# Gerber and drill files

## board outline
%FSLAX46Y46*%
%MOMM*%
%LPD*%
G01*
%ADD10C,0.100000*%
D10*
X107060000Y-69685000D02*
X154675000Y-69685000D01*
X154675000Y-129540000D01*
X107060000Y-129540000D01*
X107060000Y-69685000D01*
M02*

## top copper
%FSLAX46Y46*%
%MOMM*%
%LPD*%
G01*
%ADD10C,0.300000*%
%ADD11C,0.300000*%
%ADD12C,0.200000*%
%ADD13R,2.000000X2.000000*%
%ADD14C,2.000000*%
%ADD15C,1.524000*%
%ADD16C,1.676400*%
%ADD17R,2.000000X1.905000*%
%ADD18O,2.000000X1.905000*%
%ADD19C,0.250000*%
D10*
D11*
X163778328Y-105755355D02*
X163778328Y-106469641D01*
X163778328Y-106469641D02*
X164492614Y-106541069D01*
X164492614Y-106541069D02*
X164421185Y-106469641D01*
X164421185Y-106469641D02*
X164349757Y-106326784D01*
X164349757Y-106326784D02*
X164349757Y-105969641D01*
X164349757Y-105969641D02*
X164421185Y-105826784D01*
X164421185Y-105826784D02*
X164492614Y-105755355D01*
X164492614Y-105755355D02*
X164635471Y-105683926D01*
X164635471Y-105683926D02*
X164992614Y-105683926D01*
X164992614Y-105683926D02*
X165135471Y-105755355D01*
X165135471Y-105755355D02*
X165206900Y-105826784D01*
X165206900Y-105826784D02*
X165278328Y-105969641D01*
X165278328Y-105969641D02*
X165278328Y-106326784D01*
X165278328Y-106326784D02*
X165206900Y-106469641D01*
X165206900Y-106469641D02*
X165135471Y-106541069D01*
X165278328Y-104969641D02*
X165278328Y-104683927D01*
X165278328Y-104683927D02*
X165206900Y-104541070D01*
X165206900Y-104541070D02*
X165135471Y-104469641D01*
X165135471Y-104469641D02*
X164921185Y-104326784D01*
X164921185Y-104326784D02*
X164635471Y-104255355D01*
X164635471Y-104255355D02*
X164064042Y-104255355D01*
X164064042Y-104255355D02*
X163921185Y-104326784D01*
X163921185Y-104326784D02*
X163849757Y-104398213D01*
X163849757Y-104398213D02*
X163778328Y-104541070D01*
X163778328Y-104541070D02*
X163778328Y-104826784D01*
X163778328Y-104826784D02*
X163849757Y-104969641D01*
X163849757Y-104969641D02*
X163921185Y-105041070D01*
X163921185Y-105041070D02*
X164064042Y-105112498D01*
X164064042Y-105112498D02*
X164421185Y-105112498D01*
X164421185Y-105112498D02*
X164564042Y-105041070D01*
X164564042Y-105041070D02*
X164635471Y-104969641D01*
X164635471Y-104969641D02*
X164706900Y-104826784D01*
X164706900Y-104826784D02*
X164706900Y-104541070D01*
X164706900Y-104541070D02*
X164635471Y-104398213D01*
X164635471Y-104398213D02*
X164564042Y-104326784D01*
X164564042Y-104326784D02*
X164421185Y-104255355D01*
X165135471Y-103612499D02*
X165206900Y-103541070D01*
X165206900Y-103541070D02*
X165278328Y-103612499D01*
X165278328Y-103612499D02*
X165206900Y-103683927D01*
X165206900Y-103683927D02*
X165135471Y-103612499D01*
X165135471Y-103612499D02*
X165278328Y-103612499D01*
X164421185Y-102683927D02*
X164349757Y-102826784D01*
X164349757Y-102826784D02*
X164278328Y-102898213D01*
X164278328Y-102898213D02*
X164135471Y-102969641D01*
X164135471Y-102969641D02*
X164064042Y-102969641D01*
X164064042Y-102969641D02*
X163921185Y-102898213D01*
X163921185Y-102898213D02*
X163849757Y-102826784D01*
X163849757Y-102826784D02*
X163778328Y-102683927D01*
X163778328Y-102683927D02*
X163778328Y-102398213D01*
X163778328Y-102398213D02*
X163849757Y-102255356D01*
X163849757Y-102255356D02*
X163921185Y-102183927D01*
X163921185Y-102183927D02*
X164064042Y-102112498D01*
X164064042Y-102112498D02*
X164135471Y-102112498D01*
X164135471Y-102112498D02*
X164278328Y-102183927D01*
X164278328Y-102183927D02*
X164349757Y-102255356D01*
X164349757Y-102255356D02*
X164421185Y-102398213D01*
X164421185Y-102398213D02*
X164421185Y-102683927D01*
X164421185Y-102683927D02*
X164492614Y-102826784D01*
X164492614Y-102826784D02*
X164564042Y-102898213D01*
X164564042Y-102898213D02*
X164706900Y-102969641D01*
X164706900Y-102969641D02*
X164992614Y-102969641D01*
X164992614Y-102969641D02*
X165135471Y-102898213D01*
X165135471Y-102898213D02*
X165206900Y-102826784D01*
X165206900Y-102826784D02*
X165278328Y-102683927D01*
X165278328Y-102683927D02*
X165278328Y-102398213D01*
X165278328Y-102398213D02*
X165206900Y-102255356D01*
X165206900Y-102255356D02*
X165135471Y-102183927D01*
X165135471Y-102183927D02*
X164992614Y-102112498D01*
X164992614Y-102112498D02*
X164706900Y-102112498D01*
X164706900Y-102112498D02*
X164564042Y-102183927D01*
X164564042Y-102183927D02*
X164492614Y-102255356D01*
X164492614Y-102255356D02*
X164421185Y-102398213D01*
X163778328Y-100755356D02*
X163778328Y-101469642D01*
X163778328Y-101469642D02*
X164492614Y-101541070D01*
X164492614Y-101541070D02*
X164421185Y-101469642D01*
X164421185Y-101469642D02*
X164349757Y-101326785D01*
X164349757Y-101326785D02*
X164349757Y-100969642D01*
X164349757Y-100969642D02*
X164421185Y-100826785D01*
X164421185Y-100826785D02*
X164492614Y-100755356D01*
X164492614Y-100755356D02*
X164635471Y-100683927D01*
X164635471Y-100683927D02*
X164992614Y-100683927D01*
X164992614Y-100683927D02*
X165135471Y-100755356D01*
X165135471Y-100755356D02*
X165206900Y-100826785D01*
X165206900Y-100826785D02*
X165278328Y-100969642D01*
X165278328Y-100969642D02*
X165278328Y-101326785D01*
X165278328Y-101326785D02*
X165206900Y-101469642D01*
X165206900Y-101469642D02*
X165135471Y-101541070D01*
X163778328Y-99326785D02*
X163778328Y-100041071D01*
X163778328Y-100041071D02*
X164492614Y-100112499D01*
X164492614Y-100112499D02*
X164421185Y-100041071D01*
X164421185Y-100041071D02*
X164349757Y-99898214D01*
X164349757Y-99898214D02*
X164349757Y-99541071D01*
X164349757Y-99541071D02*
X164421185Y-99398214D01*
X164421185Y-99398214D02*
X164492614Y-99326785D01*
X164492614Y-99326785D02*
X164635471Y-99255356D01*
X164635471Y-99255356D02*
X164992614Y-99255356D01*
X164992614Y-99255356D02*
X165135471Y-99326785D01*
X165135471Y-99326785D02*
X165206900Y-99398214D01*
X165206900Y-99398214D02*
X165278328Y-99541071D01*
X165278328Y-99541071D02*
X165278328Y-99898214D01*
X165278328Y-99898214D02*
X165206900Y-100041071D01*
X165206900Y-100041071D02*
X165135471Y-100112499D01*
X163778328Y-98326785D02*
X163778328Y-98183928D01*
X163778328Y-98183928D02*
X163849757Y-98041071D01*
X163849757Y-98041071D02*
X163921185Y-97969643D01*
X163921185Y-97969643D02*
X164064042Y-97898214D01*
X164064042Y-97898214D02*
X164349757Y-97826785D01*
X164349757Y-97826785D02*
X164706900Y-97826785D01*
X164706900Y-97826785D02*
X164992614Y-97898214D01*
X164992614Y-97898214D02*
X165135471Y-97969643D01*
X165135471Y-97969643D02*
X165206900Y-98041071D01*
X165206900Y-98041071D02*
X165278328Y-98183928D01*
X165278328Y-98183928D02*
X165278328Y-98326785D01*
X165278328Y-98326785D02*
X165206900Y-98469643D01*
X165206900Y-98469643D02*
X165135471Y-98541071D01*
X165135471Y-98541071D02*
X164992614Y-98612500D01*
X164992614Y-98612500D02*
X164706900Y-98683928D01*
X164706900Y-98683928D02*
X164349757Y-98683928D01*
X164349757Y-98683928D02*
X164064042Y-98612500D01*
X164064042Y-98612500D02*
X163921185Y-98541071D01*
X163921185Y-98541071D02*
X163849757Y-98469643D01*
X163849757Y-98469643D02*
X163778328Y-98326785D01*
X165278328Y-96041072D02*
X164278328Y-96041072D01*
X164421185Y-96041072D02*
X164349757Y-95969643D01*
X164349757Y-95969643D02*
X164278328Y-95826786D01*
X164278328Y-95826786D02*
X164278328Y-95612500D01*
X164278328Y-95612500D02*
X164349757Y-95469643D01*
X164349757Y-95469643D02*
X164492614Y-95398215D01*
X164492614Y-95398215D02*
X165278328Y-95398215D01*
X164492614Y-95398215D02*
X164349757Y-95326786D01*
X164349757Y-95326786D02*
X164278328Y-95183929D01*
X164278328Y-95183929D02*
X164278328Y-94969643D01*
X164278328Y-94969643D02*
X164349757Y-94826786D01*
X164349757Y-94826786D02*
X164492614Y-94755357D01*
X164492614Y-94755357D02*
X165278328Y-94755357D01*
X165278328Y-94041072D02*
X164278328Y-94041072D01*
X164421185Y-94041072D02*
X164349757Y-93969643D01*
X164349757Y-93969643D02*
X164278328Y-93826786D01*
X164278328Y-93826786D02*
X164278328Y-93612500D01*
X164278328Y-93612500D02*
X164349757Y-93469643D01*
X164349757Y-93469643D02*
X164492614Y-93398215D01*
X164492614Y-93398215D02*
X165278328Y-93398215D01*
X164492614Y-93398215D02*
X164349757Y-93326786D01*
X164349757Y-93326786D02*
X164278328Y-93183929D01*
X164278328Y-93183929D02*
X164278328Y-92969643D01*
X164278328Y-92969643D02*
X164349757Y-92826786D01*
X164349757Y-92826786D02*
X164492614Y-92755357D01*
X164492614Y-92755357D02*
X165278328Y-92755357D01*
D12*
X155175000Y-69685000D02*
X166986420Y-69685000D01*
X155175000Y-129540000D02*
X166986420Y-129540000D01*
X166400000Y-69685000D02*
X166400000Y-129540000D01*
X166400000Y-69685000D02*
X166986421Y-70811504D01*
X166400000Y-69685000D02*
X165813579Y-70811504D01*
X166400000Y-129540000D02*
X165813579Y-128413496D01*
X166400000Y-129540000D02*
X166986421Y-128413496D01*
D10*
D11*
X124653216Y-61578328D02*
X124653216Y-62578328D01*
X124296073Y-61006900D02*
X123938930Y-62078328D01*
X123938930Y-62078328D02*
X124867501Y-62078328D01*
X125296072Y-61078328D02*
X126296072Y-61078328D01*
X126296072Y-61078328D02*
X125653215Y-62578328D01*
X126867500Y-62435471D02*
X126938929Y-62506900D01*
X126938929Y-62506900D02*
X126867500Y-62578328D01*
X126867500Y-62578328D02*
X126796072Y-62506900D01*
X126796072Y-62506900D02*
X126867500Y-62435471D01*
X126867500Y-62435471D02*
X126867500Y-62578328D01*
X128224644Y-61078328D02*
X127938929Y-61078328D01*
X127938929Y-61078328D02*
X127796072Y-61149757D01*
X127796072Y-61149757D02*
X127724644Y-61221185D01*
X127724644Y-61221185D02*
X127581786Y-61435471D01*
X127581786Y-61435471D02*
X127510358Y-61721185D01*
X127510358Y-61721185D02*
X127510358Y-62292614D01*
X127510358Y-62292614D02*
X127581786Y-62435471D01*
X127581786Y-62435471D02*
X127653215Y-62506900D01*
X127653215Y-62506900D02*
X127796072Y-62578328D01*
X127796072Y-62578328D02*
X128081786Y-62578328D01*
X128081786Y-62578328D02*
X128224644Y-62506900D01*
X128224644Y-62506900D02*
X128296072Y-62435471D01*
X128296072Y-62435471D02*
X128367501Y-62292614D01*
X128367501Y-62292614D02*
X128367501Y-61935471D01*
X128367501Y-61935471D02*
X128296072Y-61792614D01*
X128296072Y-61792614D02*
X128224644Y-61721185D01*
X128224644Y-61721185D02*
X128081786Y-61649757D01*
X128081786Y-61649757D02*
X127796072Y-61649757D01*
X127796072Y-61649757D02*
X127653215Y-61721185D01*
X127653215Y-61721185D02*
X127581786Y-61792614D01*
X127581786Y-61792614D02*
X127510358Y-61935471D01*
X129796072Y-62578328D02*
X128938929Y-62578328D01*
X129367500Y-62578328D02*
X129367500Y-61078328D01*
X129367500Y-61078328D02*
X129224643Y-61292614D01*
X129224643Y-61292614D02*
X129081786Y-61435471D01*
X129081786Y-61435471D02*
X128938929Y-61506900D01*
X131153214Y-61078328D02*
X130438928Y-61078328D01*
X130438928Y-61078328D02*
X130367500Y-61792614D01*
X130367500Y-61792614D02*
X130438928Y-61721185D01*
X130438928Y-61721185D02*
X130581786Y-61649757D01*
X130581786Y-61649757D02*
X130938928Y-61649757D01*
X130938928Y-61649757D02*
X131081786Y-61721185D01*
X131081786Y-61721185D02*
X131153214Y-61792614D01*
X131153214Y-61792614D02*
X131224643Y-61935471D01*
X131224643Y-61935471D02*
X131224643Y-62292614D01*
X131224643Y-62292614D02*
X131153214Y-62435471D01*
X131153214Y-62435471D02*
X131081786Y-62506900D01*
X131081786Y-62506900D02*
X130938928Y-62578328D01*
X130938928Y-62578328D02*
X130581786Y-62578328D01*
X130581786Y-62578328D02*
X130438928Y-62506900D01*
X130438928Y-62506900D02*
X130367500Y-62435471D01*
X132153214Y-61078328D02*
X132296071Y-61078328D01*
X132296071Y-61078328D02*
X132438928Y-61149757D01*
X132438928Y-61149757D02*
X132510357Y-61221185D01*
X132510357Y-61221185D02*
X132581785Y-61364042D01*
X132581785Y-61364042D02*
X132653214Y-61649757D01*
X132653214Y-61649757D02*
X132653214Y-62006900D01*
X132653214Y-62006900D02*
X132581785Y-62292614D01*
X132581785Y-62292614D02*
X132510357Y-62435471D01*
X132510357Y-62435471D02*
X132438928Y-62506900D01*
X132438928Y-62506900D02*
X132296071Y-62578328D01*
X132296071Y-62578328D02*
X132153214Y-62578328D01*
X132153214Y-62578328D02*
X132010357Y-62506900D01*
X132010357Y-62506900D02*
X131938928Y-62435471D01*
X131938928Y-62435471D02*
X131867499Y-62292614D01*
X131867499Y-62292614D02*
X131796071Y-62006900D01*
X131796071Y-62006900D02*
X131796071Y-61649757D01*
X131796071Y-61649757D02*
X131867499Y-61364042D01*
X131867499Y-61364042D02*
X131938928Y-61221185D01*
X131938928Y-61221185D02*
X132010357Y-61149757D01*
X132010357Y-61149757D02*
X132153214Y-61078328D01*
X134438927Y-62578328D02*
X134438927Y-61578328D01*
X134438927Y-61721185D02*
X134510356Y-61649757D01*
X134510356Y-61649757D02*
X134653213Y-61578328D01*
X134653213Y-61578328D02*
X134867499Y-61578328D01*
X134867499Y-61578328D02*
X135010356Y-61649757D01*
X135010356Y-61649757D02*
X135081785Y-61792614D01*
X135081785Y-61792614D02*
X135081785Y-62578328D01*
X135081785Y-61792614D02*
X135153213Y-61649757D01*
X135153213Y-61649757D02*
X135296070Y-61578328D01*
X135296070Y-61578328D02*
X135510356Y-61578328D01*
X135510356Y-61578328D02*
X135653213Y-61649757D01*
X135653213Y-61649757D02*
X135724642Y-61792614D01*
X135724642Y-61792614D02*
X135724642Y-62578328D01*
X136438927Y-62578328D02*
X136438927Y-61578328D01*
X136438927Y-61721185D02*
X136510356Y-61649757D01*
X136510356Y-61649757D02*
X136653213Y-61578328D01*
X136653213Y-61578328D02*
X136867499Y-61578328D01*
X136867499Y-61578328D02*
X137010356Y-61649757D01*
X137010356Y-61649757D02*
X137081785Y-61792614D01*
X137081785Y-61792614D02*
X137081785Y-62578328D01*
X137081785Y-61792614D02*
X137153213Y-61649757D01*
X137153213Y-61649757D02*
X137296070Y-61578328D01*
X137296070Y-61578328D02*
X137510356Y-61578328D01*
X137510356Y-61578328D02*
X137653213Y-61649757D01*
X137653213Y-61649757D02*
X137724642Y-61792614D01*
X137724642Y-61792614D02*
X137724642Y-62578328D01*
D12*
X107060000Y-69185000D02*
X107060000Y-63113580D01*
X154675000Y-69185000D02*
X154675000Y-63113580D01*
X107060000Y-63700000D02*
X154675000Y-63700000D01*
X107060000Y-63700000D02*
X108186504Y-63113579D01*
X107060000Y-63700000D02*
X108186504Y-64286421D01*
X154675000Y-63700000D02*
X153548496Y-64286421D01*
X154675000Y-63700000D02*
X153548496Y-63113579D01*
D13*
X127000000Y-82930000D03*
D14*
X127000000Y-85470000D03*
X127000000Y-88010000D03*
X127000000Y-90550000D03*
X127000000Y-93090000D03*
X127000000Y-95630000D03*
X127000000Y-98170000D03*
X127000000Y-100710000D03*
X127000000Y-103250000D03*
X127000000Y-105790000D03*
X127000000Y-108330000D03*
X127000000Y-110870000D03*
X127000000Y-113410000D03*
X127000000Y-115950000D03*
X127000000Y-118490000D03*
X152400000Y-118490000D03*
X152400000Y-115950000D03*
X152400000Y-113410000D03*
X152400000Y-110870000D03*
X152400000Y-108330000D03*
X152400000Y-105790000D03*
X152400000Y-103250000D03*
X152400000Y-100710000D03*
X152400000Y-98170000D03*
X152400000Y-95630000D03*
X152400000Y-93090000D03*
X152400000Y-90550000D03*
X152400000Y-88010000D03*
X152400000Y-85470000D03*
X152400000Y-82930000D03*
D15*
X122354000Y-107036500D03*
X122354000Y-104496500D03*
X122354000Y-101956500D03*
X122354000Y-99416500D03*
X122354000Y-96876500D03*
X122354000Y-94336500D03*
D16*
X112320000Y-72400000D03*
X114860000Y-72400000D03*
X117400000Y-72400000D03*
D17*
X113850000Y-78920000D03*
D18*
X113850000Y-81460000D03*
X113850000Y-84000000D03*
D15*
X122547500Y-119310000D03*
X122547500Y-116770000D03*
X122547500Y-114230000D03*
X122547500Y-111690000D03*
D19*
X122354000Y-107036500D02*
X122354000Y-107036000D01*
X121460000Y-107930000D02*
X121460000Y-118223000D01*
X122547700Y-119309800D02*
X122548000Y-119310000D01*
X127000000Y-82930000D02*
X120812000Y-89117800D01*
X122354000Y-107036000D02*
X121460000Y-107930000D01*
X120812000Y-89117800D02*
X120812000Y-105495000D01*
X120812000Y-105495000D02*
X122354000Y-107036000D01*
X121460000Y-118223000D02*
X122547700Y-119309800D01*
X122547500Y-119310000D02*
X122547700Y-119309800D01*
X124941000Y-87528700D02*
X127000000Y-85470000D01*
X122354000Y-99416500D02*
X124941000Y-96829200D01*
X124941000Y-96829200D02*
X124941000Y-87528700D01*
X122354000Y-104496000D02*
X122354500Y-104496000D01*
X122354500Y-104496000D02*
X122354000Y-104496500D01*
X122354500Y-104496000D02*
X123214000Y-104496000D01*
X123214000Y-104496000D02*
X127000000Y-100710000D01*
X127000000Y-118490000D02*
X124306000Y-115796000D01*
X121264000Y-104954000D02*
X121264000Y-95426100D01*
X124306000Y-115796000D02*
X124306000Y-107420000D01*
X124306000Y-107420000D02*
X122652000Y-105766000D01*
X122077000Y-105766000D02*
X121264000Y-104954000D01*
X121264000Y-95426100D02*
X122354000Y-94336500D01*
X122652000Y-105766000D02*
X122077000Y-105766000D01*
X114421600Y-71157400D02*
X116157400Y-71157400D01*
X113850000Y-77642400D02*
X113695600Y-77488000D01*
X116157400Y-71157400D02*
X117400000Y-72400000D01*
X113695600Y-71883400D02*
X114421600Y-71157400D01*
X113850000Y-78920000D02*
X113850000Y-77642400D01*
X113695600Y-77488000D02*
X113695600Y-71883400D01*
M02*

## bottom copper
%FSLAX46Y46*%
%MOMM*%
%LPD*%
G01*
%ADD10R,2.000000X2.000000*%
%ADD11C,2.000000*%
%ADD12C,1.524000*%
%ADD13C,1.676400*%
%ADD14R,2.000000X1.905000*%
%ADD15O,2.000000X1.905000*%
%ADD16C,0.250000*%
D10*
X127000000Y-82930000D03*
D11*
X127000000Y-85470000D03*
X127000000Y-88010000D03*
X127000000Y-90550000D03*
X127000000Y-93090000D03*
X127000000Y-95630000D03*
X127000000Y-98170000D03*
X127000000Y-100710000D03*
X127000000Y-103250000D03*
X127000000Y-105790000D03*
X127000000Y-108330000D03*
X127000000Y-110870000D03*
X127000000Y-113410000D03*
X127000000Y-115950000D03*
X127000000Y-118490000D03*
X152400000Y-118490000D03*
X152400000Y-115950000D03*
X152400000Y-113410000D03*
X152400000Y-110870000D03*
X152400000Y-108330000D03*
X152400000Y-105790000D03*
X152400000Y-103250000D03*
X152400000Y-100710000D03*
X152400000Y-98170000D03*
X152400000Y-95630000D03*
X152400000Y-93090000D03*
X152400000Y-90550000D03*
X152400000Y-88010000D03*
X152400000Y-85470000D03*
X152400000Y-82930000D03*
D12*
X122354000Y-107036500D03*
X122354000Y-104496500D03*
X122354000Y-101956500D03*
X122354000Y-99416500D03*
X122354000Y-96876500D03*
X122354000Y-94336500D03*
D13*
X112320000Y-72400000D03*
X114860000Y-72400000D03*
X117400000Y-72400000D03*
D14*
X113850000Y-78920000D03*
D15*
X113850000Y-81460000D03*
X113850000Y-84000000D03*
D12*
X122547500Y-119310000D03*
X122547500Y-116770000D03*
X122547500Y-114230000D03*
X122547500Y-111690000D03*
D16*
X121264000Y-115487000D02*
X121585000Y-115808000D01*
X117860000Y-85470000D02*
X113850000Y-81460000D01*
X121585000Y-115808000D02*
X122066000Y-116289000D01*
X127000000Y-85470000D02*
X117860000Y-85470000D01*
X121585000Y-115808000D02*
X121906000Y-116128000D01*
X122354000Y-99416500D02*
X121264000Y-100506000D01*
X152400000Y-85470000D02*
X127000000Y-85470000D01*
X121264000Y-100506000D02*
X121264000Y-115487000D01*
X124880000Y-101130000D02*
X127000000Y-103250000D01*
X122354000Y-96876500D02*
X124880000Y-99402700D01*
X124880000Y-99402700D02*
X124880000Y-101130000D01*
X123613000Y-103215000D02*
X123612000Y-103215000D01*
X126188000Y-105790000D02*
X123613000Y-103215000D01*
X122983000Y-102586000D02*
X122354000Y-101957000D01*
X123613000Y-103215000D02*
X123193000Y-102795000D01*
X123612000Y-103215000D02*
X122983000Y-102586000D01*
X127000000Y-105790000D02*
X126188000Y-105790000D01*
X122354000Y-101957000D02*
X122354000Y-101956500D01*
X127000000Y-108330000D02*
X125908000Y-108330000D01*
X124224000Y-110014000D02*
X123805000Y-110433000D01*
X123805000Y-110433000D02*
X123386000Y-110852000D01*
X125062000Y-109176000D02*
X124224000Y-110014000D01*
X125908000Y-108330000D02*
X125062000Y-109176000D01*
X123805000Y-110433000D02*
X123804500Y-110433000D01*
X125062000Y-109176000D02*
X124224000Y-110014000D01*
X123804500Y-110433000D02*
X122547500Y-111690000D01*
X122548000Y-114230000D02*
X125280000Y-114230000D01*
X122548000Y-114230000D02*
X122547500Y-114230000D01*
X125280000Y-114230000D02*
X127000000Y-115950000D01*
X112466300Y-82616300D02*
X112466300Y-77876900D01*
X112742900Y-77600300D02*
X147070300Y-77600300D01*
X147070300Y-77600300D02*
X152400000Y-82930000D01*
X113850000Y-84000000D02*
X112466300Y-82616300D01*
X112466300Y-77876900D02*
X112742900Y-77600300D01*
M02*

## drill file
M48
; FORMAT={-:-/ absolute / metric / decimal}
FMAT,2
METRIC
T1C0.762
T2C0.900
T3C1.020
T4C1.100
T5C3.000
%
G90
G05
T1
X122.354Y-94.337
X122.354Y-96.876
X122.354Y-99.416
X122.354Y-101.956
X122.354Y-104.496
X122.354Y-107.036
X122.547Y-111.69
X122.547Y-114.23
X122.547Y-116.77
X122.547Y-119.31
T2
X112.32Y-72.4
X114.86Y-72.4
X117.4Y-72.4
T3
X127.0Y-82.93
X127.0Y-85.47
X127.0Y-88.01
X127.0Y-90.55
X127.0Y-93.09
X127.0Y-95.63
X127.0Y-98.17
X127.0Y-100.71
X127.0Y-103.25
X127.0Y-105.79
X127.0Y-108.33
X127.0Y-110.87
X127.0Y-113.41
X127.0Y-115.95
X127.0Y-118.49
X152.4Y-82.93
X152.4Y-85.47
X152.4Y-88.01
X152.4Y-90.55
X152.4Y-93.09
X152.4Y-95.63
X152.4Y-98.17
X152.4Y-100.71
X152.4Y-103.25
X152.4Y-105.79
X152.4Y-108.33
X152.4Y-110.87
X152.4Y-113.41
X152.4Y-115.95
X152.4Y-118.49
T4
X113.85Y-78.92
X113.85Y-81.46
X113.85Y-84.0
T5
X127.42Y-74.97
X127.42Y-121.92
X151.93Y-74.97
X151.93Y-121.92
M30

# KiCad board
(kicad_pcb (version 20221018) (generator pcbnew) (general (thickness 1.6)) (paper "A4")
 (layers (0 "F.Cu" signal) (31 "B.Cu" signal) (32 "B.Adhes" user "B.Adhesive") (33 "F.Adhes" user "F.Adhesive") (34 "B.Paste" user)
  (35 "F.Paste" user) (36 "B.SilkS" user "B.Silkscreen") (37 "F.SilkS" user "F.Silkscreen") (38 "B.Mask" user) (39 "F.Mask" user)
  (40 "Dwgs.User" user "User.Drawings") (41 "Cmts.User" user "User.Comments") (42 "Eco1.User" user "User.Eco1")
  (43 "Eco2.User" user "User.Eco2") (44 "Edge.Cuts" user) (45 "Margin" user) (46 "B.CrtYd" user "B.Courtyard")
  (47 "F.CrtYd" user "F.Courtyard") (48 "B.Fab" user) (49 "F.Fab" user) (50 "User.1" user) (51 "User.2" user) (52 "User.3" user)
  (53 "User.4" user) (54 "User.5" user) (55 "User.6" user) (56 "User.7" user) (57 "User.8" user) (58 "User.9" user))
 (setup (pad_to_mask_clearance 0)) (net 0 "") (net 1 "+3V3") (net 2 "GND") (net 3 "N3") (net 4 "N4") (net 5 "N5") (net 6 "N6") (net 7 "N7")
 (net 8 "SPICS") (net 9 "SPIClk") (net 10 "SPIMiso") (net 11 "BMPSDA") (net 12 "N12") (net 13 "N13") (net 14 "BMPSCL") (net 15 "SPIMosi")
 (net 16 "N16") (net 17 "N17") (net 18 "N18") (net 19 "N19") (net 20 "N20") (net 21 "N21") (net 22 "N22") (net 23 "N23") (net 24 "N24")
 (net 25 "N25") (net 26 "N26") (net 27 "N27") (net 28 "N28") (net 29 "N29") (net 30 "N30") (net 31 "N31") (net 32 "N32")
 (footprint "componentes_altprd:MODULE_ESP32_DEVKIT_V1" (layer "F.Cu") (at 139.7 98.445)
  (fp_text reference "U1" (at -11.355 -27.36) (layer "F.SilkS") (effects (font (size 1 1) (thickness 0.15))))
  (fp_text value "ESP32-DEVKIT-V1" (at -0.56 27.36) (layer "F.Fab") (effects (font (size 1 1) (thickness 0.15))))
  (pad "" np_thru_hole circle (at -12.28 -23.475) (size 3 3) (drill 3) (layers "*.Cu" "*.Mask"))
  (pad "" np_thru_hole circle (at -12.28 23.475) (size 3 3) (drill 3) (layers "*.Cu" "*.Mask"))
  (pad "" np_thru_hole circle (at 12.23 -23.475) (size 3 3) (drill 3) (layers "*.Cu" "*.Mask"))
  (pad "" np_thru_hole circle (at 12.23 23.475) (size 3 3) (drill 3) (layers "*.Cu" "*.Mask"))
  (pad "1" thru_hole rect (at -12.7 -15.515) (size 2 2) (drill 1.02) (layers "*.Cu" "*.Mask") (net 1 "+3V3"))
  (pad "2" thru_hole circle (at -12.7 -12.975) (size 2 2) (drill 1.02) (layers "*.Cu" "*.Mask") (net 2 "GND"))
  (pad "3" thru_hole circle (at -12.7 -10.435) (size 2 2) (drill 1.02) (layers "*.Cu" "*.Mask") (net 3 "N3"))
  (pad "4" thru_hole circle (at -12.7 -7.895) (size 2 2) (drill 1.02) (layers "*.Cu" "*.Mask") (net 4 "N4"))
  (pad "5" thru_hole circle (at -12.7 -5.355) (size 2 2) (drill 1.02) (layers "*.Cu" "*.Mask") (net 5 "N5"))
  (pad "6" thru_hole circle (at -12.7 -2.815) (size 2 2) (drill 1.02) (layers "*.Cu" "*.Mask") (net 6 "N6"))
  (pad "7" thru_hole circle (at -12.7 -0.275) (size 2 2) (drill 1.02) (layers "*.Cu" "*.Mask") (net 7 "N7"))
  (pad "8" thru_hole circle (at -12.7 2.265) (size 2 2) (drill 1.02) (layers "*.Cu" "*.Mask") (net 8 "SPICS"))
  (pad "9" thru_hole circle (at -12.7 4.805) (size 2 2) (drill 1.02) (layers "*.Cu" "*.Mask") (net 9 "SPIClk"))
  (pad "10" thru_hole circle (at -12.7 7.345) (size 2 2) (drill 1.02) (layers "*.Cu" "*.Mask") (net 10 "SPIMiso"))
  (pad "11" thru_hole circle (at -12.7 9.885) (size 2 2) (drill 1.02) (layers "*.Cu" "*.Mask") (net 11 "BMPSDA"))
  (pad "12" thru_hole circle (at -12.7 12.425) (size 2 2) (drill 1.02) (layers "*.Cu" "*.Mask") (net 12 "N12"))
  (pad "13" thru_hole circle (at -12.7 14.965) (size 2 2) (drill 1.02) (layers "*.Cu" "*.Mask") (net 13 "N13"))
  (pad "14" thru_hole circle (at -12.7 17.505) (size 2 2) (drill 1.02) (layers "*.Cu" "*.Mask") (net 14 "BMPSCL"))
  (pad "15" thru_hole circle (at -12.7 20.045) (size 2 2) (drill 1.02) (layers "*.Cu" "*.Mask") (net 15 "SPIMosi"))
  (pad "16" thru_hole circle (at 12.7 20.045) (size 2 2) (drill 1.02) (layers "*.Cu" "*.Mask") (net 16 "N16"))
  (pad "17" thru_hole circle (at 12.7 17.505) (size 2 2) (drill 1.02) (layers "*.Cu" "*.Mask") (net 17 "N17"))
  (pad "18" thru_hole circle (at 12.7 14.965) (size 2 2) (drill 1.02) (layers "*.Cu" "*.Mask") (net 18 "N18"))
  (pad "19" thru_hole circle (at 12.7 12.425) (size 2 2) (drill 1.02) (layers "*.Cu" "*.Mask") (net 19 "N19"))
  (pad "20" thru_hole circle (at 12.7 9.885) (size 2 2) (drill 1.02) (layers "*.Cu" "*.Mask") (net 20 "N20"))
  (pad "21" thru_hole circle (at 12.7 7.345) (size 2 2) (drill 1.02) (layers "*.Cu" "*.Mask") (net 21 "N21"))
  (pad "22" thru_hole circle (at 12.7 4.805) (size 2 2) (drill 1.02) (layers "*.Cu" "*.Mask") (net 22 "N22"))
  (pad "23" thru_hole circle (at 12.7 2.265) (size 2 2) (drill 1.02) (layers "*.Cu" "*.Mask") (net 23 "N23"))
  (pad "24" thru_hole circle (at 12.7 -0.275) (size 2 2) (drill 1.02) (layers "*.Cu" "*.Mask") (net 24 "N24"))
  (pad "25" thru_hole circle (at 12.7 -2.815) (size 2 2) (drill 1.02) (layers "*.Cu" "*.Mask") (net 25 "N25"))
  (pad "26" thru_hole circle (at 12.7 -5.355) (size 2 2) (drill 1.02) (layers "*.Cu" "*.Mask") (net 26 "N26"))
  (pad "27" thru_hole circle (at 12.7 -7.895) (size 2 2) (drill 1.02) (layers "*.Cu" "*.Mask") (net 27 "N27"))
  (pad "28" thru_hole circle (at 12.7 -10.435) (size 2 2) (drill 1.02) (layers "*.Cu" "*.Mask") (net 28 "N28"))
  (pad "29" thru_hole circle (at 12.7 -12.975) (size 2 2) (drill 1.02) (layers "*.Cu" "*.Mask") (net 2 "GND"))
  (pad "30" thru_hole circle (at 12.7 -15.515) (size 2 2) (drill 1.02) (layers "*.Cu" "*.Mask") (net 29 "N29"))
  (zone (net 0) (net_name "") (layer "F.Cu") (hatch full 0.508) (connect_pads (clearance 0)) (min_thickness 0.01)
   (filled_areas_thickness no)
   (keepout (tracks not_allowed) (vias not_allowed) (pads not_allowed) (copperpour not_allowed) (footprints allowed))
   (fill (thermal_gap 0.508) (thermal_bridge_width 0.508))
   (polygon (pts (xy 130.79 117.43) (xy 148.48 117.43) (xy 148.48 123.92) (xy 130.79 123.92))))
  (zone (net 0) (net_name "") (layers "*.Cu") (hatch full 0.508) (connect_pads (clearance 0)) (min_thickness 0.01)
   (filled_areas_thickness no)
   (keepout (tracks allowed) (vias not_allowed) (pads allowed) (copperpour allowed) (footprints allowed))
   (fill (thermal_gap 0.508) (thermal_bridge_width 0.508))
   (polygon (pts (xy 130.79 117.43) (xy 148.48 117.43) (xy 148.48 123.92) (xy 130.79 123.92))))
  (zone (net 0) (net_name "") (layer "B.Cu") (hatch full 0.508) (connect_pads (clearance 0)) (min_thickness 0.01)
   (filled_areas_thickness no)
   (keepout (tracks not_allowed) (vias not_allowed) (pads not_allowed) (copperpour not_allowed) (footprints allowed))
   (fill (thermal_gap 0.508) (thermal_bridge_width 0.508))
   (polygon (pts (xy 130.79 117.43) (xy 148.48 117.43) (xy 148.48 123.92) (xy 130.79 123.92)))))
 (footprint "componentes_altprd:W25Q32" (layer "F.Cu") (at 115.4325 101.0675 180)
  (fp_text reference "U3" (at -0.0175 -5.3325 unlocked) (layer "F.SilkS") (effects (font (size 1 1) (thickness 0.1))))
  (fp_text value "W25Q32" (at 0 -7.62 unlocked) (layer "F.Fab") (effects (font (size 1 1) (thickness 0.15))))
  (pad "1" thru_hole circle (at -6.9215 -5.969 180) (size 1.524 1.524) (drill 0.762) (layers "*.Cu" "*.Mask") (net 1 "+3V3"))
  (pad "2" thru_hole circle (at -6.9215 -3.429 180) (size 1.524 1.524) (drill 0.762) (layers "*.Cu" "*.Mask") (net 8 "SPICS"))
  (pad "3" thru_hole circle (at -6.9215 -0.889 180) (size 1.524 1.524) (drill 0.762) (layers "*.Cu" "*.Mask") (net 10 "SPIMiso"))
  (pad "4" thru_hole circle (at -6.9215 1.651 180) (size 1.524 1.524) (drill 0.762) (layers "*.Cu" "*.Mask") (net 2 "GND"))
  (pad "5" thru_hole circle (at -6.9215 4.191 180) (size 1.524 1.524) (drill 0.762) (layers "*.Cu" "*.Mask") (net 9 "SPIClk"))
  (pad "6" thru_hole circle (at -6.9215 6.731 180) (size 1.524 1.524) (drill 0.762) (layers "*.Cu" "*.Mask") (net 15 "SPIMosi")))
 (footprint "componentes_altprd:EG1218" (layer "F.Cu") (at 114.86 72.4)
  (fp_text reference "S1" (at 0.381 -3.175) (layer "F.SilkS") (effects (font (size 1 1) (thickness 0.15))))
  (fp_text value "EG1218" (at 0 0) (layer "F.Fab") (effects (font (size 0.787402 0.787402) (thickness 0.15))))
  (pad "O" thru_hole circle (at -2.54 0) (size 1.6764 1.6764) (drill 0.9) (layers "*.Cu" "*.Mask") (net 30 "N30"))
  (pad "P" thru_hole circle (at 0 0) (size 1.6764 1.6764) (drill 0.9) (layers "*.Cu" "*.Mask") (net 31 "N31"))
  (pad "S" thru_hole circle (at 2.54 0) (size 1.6764 1.6764) (drill 0.9) (layers "*.Cu" "*.Mask") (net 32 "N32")))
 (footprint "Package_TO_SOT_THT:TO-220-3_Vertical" (layer "F.Cu") (at 113.85 78.92 -90)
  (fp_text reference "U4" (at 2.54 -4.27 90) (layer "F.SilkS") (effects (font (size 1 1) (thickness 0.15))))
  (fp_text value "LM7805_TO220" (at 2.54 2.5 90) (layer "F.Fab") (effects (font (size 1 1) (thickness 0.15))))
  (pad "1" thru_hole rect (at 0 0 270) (size 1.905 2) (drill 1.1) (layers "*.Cu" "*.Mask") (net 32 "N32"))
  (pad "2" thru_hole oval (at 2.54 0 270) (size 1.905 2) (drill 1.1) (layers "*.Cu" "*.Mask") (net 2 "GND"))
  (pad "3" thru_hole oval (at 5.08 0 270) (size 1.905 2) (drill 1.1) (layers "*.Cu" "*.Mask") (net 29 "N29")))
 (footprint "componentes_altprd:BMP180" (layer "F.Cu") (at 118.1025 114.23 180)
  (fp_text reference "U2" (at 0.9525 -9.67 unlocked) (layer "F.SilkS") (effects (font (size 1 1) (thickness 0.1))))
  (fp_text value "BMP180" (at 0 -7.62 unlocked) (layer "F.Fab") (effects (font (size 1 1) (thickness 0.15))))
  (pad "1" thru_hole circle (at -4.445 -5.08 180) (size 1.524 1.524) (drill 0.762) (layers "*.Cu" "*.Mask") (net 1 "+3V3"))
  (pad "2" thru_hole circle (at -4.445 -2.54 180) (size 1.524 1.524) (drill 0.762) (layers "*.Cu" "*.Mask") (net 2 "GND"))
  (pad "3" thru_hole circle (at -4.445 0 180) (size 1.524 1.524) (drill 0.762) (layers "*.Cu" "*.Mask") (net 14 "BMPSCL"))
  (pad "4" thru_hole circle (at -4.445 2.54 180) (size 1.524 1.524) (drill 0.762) (layers "*.Cu" "*.Mask") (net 11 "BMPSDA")))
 (gr_rect (start 107.06 69.685) (end 154.675 129.54) (stroke (width 0.1) (type default)) (fill none) (layer "Edge.Cuts"))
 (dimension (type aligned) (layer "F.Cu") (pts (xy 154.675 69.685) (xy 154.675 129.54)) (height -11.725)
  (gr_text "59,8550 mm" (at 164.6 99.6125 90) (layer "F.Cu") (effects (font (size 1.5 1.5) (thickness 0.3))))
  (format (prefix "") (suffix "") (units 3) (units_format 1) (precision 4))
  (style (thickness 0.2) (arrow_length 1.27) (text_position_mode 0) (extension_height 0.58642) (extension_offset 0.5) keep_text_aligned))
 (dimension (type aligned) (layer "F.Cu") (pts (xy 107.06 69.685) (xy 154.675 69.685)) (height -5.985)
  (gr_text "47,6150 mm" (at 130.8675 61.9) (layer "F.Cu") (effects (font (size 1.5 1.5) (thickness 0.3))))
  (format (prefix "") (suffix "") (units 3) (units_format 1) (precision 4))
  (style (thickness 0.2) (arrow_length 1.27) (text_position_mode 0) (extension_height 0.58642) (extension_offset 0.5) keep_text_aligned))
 (segment (start 122.354 107.0365) (end 122.354 107.036) (width 0.25) (layer "F.Cu") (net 1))
 (segment (start 121.46 107.93) (end 121.46 118.223) (width 0.25) (layer "F.Cu") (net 1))
 (segment (start 122.5477 119.3098) (end 122.548 119.31) (width 0.25) (layer "F.Cu") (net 1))
 (segment (start 127 82.93) (end 120.812 89.1178) (width 0.25) (layer "F.Cu") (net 1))
 (segment (start 122.354 107.036) (end 121.46 107.93) (width 0.25) (layer "F.Cu") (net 1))
 (segment (start 120.812 89.1178) (end 120.812 105.495) (width 0.25) (layer "F.Cu") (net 1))
 (segment (start 120.812 105.495) (end 122.354 107.036) (width 0.25) (layer "F.Cu") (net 1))
 (segment (start 121.46 118.223) (end 122.5477 119.3098) (width 0.25) (layer "F.Cu") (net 1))
 (segment (start 122.5475 119.31) (end 122.5477 119.3098) (width 0.25) (layer "F.Cu") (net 1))
 (segment (start 124.941 87.5287) (end 127 85.47) (width 0.25) (layer "F.Cu") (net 2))
 (segment (start 122.354 99.4165) (end 124.941 96.8292) (width 0.25) (layer "F.Cu") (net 2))
 (segment (start 124.941 96.8292) (end 124.941 87.5287) (width 0.25) (layer "F.Cu") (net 2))
 (segment (start 121.264 115.487) (end 121.585 115.808) (width 0.25) (layer "B.Cu") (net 2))
 (segment (start 117.86 85.47) (end 113.85 81.46) (width 0.25) (layer "B.Cu") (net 2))
 (segment (start 121.585 115.808) (end 122.066 116.289) (width 0.25) (layer "B.Cu") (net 2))
 (segment (start 127 85.47) (end 117.86 85.47) (width 0.25) (layer "B.Cu") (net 2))
 (segment (start 121.585 115.808) (end 121.906 116.128) (width 0.25) (layer "B.Cu") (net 2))
 (segment (start 122.354 99.4165) (end 121.264 100.506) (width 0.25) (layer "B.Cu") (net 2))
 (segment (start 152.4 85.47) (end 127 85.47) (width 0.25) (layer "B.Cu") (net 2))
 (segment (start 121.264 100.506) (end 121.264 115.487) (width 0.25) (layer "B.Cu") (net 2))
 (segment (start 122.354 104.496) (end 122.3545 104.496) (width 0.25) (layer "F.Cu") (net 8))
 (segment (start 122.3545 104.496) (end 122.354 104.4965) (width 0.25) (layer "F.Cu") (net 8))
 (segment (start 122.3545 104.496) (end 123.214 104.496) (width 0.25) (layer "F.Cu") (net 8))
 (segment (start 123.214 104.496) (end 127 100.71) (width 0.25) (layer "F.Cu") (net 8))
 (segment (start 124.88 101.13) (end 127 103.25) (width 0.25) (layer "B.Cu") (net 9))
 (segment (start 122.354 96.8765) (end 124.88 99.4027) (width 0.25) (layer "B.Cu") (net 9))
 (segment (start 124.88 99.4027) (end 124.88 101.13) (width 0.25) (layer "B.Cu") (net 9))
 (segment (start 123.613 103.215) (end 123.612 103.215) (width 0.25) (layer "B.Cu") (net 10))
 (segment (start 126.188 105.79) (end 123.613 103.215) (width 0.25) (layer "B.Cu") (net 10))
 (segment (start 122.983 102.586) (end 122.354 101.957) (width 0.25) (layer "B.Cu") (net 10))
 (segment (start 123.613 103.215) (end 123.193 102.795) (width 0.25) (layer "B.Cu") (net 10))
 (segment (start 123.612 103.215) (end 122.983 102.586) (width 0.25) (layer "B.Cu") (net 10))
 (segment (start 127 105.79) (end 126.188 105.79) (width 0.25) (layer "B.Cu") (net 10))
 (segment (start 122.354 101.957) (end 122.354 101.9565) (width 0.25) (layer "B.Cu") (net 10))
 (segment (start 127 108.33) (end 125.908 108.33) (width 0.25) (layer "B.Cu") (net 11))
 (segment (start 124.224 110.014) (end 123.805 110.433) (width 0.25) (layer "B.Cu") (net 11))
 (segment (start 123.805 110.433) (end 123.386 110.852) (width 0.25) (layer "B.Cu") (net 11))
 (segment (start 125.062 109.176) (end 124.224 110.014) (width 0.25) (layer "B.Cu") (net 11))
 (segment (start 125.908 108.33) (end 125.062 109.176) (width 0.25) (layer "B.Cu") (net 11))
 (segment (start 123.805 110.433) (end 123.8045 110.433) (width 0.25) (layer "B.Cu") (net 11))
 (segment (start 125.062 109.176) (end 124.224 110.014) (width 0.25) (layer "B.Cu") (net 11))
 (segment (start 123.8045 110.433) (end 122.5475 111.69) (width 0.25) (layer "B.Cu") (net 11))
 (segment (start 122.548 114.23) (end 125.28 114.23) (width 0.25) (layer "B.Cu") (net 14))
 (segment (start 122.548 114.23) (end 122.5475 114.23) (width 0.25) (layer "B.Cu") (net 14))
 (segment (start 125.28 114.23) (end 127 115.95) (width 0.25) (layer "B.Cu") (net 14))
 (segment (start 127 118.49) (end 124.306 115.796) (width 0.25) (layer "F.Cu") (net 15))
 (segment (start 121.264 104.954) (end 121.264 95.4261) (width 0.25) (layer "F.Cu") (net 15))
 (segment (start 124.306 115.796) (end 124.306 107.42) (width 0.25) (layer "F.Cu") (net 15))
 (segment (start 124.306 107.42) (end 122.652 105.766) (width 0.25) (layer "F.Cu") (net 15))
 (segment (start 122.077 105.766) (end 121.264 104.954) (width 0.25) (layer "F.Cu") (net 15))
 (segment (start 121.264 95.4261) (end 122.354 94.3365) (width 0.25) (layer "F.Cu") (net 15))
 (segment (start 122.652 105.766) (end 122.077 105.766) (width 0.25) (layer "F.Cu") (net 15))
 (segment (start 114.4216 71.1574) (end 116.1574 71.1574) (width 0.25) (layer "F.Cu") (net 32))
 (segment (start 113.85 77.6424) (end 113.6956 77.488) (width 0.25) (layer "F.Cu") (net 32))
 (segment (start 116.1574 71.1574) (end 117.4 72.4) (width 0.25) (layer "F.Cu") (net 32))
 (segment (start 113.6956 71.8834) (end 114.4216 71.1574) (width 0.25) (layer "F.Cu") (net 32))
 (segment (start 113.85 78.92) (end 113.85 77.6424) (width 0.25) (layer "F.Cu") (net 32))
 (segment (start 113.6956 77.488) (end 113.6956 71.8834) (width 0.25) (layer "F.Cu") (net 32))
 (segment (start 112.4663 82.6163) (end 112.4663 77.8769) (width 0.25) (layer "B.Cu") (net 29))
 (segment (start 112.7429 77.6003) (end 147.0703 77.6003) (width 0.25) (layer "B.Cu") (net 29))
 (segment (start 147.0703 77.6003) (end 152.4 82.93) (width 0.25) (layer "B.Cu") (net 29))
 (segment (start 113.85 84) (end 112.4663 82.6163) (width 0.25) (layer "B.Cu") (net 29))
 (segment (start 112.4663 77.8769) (end 112.7429 77.6003) (width 0.25) (layer "B.Cu") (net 29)))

